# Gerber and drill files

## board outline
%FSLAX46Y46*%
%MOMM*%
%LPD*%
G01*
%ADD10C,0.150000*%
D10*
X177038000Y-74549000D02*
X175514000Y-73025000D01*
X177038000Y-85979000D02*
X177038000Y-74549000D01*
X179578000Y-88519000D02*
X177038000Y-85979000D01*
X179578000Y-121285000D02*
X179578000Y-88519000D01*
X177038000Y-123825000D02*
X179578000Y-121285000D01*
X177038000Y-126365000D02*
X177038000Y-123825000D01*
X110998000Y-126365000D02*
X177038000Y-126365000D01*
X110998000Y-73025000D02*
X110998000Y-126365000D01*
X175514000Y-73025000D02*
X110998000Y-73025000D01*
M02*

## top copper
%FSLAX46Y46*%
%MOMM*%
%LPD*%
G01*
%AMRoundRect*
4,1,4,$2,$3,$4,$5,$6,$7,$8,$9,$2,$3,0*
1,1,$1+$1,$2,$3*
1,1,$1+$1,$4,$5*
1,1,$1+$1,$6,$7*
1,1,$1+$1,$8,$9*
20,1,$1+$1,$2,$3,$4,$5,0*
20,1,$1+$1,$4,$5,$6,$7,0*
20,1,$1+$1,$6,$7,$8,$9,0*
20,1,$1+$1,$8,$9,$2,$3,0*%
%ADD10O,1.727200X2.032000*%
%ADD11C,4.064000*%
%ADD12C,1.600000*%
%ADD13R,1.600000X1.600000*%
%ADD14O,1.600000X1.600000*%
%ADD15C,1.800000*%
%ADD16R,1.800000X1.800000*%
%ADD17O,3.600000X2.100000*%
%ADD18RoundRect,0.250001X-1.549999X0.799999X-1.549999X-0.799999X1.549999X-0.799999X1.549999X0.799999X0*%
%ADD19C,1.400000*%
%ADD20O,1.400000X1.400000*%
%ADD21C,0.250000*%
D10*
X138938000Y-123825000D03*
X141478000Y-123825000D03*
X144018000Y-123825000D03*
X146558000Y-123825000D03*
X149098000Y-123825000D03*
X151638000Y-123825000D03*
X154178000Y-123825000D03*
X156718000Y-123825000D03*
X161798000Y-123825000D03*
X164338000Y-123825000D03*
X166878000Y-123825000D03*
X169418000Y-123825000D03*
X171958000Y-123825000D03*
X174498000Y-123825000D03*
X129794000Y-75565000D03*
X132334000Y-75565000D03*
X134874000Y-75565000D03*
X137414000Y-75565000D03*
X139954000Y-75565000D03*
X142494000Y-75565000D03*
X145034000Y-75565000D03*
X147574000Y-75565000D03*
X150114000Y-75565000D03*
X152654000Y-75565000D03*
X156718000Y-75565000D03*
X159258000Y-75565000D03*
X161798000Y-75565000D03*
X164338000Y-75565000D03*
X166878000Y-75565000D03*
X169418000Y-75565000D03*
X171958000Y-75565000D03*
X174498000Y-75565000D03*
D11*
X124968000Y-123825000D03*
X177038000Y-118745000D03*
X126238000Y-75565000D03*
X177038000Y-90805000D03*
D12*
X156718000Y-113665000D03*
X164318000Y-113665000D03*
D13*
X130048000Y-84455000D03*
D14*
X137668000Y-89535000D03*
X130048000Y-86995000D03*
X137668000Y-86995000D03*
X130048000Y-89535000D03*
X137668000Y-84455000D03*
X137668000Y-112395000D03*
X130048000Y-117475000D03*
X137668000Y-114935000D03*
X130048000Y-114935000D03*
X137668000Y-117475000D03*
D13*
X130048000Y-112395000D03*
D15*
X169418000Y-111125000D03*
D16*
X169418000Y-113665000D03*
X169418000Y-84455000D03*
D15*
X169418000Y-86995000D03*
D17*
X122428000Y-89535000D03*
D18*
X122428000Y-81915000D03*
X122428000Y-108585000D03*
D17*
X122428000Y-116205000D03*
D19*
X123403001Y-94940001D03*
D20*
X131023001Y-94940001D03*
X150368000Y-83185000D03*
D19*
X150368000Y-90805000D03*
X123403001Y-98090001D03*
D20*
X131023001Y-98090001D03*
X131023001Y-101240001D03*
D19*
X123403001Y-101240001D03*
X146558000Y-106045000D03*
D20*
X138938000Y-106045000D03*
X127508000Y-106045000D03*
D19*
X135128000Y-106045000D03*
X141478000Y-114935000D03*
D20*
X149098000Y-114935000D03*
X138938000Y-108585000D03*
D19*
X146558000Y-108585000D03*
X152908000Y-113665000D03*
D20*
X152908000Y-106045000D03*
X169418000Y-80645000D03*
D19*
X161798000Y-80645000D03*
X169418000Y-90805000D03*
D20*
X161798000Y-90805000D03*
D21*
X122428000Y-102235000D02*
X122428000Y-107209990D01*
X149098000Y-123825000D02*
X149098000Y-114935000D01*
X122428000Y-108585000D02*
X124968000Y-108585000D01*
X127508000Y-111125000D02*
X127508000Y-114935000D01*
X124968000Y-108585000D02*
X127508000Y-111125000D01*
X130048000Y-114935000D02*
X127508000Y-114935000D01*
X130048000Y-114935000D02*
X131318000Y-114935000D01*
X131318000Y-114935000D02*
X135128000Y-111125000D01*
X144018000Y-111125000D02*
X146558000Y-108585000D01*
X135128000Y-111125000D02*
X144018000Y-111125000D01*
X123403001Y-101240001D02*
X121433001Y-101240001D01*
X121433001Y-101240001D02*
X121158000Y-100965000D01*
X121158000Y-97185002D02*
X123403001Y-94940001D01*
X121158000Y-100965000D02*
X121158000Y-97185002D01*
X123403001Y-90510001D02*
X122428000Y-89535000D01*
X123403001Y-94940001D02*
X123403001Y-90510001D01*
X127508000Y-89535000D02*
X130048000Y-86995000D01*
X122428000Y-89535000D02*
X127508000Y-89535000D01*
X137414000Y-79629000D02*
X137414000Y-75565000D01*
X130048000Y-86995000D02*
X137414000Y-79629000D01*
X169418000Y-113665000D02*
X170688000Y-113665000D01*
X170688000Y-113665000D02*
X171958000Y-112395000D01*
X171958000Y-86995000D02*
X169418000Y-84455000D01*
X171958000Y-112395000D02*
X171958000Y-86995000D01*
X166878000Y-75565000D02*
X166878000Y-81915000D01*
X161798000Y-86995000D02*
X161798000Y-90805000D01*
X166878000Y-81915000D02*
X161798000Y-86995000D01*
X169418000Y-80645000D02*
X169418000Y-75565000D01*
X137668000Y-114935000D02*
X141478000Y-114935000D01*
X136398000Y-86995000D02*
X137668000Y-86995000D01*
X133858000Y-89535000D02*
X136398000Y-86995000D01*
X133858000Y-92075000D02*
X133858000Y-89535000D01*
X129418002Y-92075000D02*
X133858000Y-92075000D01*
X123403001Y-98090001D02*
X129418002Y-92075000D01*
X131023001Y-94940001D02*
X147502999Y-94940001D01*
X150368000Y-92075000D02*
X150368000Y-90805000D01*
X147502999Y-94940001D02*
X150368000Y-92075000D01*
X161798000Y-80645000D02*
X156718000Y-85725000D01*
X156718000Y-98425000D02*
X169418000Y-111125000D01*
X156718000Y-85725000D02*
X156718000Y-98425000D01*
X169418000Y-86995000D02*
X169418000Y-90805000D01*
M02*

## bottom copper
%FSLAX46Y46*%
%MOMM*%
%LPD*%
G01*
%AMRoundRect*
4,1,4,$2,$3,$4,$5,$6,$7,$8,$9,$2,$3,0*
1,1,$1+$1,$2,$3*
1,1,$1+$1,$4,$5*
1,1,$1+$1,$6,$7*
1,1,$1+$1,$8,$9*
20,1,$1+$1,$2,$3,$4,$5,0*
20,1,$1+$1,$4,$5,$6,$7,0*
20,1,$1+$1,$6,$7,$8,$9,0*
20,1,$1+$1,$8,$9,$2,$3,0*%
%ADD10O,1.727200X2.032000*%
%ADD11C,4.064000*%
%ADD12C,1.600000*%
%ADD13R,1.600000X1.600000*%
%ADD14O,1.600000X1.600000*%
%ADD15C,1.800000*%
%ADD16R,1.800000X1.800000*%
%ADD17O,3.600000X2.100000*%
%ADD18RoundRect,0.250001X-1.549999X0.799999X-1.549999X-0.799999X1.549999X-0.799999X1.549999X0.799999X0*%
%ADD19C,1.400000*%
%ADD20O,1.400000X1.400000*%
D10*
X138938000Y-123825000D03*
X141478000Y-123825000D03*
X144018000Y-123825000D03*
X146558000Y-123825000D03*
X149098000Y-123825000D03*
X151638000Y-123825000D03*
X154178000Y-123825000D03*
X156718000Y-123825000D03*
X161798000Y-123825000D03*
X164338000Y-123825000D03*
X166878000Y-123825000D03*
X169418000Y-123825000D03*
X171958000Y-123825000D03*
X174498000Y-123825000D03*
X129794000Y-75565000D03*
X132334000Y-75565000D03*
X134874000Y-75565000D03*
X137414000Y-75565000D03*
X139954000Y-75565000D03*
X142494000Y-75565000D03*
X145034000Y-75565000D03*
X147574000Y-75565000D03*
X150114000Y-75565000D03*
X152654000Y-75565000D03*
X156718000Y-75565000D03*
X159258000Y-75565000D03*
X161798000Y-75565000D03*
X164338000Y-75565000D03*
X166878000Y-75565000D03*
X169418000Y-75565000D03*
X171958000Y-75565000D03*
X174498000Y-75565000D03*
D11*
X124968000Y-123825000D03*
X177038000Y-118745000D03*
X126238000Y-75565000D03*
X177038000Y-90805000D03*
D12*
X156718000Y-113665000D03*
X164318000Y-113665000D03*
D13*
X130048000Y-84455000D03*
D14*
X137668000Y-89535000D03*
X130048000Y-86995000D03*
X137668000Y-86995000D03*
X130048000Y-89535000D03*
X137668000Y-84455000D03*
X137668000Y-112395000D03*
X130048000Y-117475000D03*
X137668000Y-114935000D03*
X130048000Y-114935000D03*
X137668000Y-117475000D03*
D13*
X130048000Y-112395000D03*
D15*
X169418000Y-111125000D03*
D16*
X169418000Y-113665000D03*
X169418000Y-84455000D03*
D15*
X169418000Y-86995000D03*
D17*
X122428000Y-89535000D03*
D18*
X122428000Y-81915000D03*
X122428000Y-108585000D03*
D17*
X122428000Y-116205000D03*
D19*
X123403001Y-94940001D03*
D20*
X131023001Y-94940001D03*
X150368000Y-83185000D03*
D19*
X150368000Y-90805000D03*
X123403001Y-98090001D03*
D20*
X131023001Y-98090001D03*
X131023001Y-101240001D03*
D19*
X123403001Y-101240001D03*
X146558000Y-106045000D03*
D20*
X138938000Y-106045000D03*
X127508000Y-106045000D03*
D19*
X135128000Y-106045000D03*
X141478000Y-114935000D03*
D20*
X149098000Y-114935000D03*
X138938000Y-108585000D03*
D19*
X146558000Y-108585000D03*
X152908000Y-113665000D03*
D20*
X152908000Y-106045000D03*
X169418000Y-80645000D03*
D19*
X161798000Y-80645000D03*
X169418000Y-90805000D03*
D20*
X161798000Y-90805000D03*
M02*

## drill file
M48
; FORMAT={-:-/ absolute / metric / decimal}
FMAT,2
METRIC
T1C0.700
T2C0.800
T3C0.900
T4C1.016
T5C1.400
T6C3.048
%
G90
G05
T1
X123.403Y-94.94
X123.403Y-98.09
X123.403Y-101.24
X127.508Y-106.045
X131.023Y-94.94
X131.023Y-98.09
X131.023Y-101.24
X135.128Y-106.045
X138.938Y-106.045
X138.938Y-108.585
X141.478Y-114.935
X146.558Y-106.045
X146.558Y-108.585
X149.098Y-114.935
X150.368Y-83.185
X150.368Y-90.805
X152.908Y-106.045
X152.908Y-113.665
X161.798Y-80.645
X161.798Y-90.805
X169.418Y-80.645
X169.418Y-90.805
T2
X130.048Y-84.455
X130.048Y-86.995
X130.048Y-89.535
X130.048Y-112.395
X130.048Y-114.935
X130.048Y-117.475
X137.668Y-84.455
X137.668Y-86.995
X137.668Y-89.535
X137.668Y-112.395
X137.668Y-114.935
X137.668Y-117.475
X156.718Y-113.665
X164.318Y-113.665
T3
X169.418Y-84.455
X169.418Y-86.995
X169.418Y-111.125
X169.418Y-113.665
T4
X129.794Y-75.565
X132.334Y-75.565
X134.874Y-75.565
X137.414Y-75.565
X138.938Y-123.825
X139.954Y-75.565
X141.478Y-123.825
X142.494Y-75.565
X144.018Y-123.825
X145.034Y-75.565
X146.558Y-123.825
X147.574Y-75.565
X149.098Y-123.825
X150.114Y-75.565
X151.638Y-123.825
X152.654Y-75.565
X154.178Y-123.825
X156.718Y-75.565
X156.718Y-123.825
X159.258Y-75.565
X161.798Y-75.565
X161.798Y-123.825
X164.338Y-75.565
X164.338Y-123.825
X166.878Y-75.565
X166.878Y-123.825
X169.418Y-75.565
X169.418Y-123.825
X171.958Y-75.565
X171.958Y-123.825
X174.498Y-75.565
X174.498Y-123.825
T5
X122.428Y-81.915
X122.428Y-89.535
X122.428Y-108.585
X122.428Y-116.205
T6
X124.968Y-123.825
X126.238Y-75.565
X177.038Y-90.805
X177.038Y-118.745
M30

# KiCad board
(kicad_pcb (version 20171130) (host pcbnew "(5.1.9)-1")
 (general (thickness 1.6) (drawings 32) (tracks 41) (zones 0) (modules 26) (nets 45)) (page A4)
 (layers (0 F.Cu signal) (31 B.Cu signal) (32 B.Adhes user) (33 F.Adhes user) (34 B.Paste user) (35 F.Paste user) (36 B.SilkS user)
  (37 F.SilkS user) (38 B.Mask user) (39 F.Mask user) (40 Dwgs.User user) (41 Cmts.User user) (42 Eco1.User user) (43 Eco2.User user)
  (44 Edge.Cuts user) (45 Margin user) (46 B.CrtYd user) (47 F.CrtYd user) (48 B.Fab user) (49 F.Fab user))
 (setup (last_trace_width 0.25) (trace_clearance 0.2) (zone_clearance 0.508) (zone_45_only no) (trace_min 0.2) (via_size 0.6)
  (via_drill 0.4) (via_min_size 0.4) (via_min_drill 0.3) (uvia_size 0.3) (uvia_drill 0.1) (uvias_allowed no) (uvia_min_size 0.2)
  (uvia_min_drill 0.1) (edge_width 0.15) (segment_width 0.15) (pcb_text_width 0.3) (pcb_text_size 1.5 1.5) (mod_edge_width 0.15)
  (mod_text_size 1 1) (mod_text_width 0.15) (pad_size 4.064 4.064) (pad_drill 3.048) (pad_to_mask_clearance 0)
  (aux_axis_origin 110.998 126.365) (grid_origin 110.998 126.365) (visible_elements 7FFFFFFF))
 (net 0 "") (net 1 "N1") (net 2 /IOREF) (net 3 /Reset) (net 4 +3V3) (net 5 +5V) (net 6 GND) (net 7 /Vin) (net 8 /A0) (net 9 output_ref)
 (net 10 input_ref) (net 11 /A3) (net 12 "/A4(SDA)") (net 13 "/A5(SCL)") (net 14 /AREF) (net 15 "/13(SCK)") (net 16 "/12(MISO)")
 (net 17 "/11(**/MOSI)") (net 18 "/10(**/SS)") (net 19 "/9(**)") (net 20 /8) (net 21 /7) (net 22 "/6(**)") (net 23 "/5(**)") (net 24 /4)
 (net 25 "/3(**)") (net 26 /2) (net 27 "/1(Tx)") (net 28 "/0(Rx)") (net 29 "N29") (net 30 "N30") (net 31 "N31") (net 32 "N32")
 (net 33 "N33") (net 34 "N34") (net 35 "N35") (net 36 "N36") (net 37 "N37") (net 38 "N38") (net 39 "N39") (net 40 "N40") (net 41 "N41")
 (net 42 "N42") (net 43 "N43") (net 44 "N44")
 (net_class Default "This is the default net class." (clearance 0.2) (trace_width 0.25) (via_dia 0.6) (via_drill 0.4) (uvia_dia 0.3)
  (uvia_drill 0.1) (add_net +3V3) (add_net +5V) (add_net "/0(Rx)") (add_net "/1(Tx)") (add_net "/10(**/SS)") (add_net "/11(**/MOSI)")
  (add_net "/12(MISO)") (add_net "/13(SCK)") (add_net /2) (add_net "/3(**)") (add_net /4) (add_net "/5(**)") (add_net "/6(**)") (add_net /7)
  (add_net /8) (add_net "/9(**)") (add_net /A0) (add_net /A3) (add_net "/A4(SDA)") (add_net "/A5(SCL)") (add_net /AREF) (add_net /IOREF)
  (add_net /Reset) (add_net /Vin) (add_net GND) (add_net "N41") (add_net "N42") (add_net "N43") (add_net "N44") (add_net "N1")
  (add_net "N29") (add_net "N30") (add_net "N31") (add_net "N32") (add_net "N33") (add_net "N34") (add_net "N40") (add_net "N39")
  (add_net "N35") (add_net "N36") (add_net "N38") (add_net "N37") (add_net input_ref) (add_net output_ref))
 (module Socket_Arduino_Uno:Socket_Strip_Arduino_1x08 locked (layer F.Cu) (at 138.938 123.825)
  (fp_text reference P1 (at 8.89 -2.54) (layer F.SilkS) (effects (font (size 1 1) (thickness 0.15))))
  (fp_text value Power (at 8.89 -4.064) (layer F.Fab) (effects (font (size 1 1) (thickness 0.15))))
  (pad 1 thru_hole oval (at 0 0) (size 1.7272 2.032) (drill 1.016) (layers *.Cu *.Mask F.SilkS) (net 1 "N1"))
  (pad 2 thru_hole oval (at 2.54 0) (size 1.7272 2.032) (drill 1.016) (layers *.Cu *.Mask F.SilkS) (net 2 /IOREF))
  (pad 3 thru_hole oval (at 5.08 0) (size 1.7272 2.032) (drill 1.016) (layers *.Cu *.Mask F.SilkS) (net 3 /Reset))
  (pad 4 thru_hole oval (at 7.62 0) (size 1.7272 2.032) (drill 1.016) (layers *.Cu *.Mask F.SilkS) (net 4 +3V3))
  (pad 5 thru_hole oval (at 10.16 0) (size 1.7272 2.032) (drill 1.016) (layers *.Cu *.Mask F.SilkS) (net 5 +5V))
  (pad 6 thru_hole oval (at 12.7 0) (size 1.7272 2.032) (drill 1.016) (layers *.Cu *.Mask F.SilkS) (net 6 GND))
  (pad 7 thru_hole oval (at 15.24 0) (size 1.7272 2.032) (drill 1.016) (layers *.Cu *.Mask F.SilkS) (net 6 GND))
  (pad 8 thru_hole oval (at 17.78 0) (size 1.7272 2.032) (drill 1.016) (layers *.Cu *.Mask F.SilkS) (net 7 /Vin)))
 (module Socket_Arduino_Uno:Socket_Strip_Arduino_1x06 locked (layer F.Cu) (at 161.798 123.825)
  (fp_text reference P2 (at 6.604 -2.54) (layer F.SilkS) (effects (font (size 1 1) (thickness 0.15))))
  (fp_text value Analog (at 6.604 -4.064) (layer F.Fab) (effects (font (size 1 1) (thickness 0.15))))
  (pad 1 thru_hole oval (at 0 0) (size 1.7272 2.032) (drill 1.016) (layers *.Cu *.Mask F.SilkS) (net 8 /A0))
  (pad 2 thru_hole oval (at 2.54 0) (size 1.7272 2.032) (drill 1.016) (layers *.Cu *.Mask F.SilkS) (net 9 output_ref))
  (pad 3 thru_hole oval (at 5.08 0) (size 1.7272 2.032) (drill 1.016) (layers *.Cu *.Mask F.SilkS) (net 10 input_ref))
  (pad 4 thru_hole oval (at 7.62 0) (size 1.7272 2.032) (drill 1.016) (layers *.Cu *.Mask F.SilkS) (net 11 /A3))
  (pad 5 thru_hole oval (at 10.16 0) (size 1.7272 2.032) (drill 1.016) (layers *.Cu *.Mask F.SilkS) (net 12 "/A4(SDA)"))
  (pad 6 thru_hole oval (at 12.7 0) (size 1.7272 2.032) (drill 1.016) (layers *.Cu *.Mask F.SilkS) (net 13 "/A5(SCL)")))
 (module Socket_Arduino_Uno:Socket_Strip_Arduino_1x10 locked (layer F.Cu) (at 129.794 75.565)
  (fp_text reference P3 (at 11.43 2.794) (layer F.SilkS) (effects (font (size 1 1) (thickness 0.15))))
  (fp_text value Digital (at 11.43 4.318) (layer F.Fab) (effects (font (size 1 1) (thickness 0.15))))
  (pad 1 thru_hole oval (at 0 0) (size 1.7272 2.032) (drill 1.016) (layers *.Cu *.Mask F.SilkS) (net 13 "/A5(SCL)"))
  (pad 2 thru_hole oval (at 2.54 0) (size 1.7272 2.032) (drill 1.016) (layers *.Cu *.Mask F.SilkS) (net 12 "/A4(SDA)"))
  (pad 3 thru_hole oval (at 5.08 0) (size 1.7272 2.032) (drill 1.016) (layers *.Cu *.Mask F.SilkS) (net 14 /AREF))
  (pad 4 thru_hole oval (at 7.62 0) (size 1.7272 2.032) (drill 1.016) (layers *.Cu *.Mask F.SilkS) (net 6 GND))
  (pad 5 thru_hole oval (at 10.16 0) (size 1.7272 2.032) (drill 1.016) (layers *.Cu *.Mask F.SilkS) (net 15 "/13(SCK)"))
  (pad 6 thru_hole oval (at 12.7 0) (size 1.7272 2.032) (drill 1.016) (layers *.Cu *.Mask F.SilkS) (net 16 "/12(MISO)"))
  (pad 7 thru_hole oval (at 15.24 0) (size 1.7272 2.032) (drill 1.016) (layers *.Cu *.Mask F.SilkS) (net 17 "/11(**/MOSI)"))
  (pad 8 thru_hole oval (at 17.78 0) (size 1.7272 2.032) (drill 1.016) (layers *.Cu *.Mask F.SilkS) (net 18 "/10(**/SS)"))
  (pad 9 thru_hole oval (at 20.32 0) (size 1.7272 2.032) (drill 1.016) (layers *.Cu *.Mask F.SilkS) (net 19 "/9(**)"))
  (pad 10 thru_hole oval (at 22.86 0) (size 1.7272 2.032) (drill 1.016) (layers *.Cu *.Mask F.SilkS) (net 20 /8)))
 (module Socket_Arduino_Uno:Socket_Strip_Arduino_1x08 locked (layer F.Cu) (at 156.718 75.565)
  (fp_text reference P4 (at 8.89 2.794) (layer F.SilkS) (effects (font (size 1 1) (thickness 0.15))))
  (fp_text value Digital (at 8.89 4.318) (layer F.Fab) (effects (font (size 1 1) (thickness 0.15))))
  (pad 1 thru_hole oval (at 0 0) (size 1.7272 2.032) (drill 1.016) (layers *.Cu *.Mask F.SilkS) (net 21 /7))
  (pad 2 thru_hole oval (at 2.54 0) (size 1.7272 2.032) (drill 1.016) (layers *.Cu *.Mask F.SilkS) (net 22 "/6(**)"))
  (pad 3 thru_hole oval (at 5.08 0) (size 1.7272 2.032) (drill 1.016) (layers *.Cu *.Mask F.SilkS) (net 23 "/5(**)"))
  (pad 4 thru_hole oval (at 7.62 0) (size 1.7272 2.032) (drill 1.016) (layers *.Cu *.Mask F.SilkS) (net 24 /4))
  (pad 5 thru_hole oval (at 10.16 0) (size 1.7272 2.032) (drill 1.016) (layers *.Cu *.Mask F.SilkS) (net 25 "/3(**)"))
  (pad 6 thru_hole oval (at 12.7 0) (size 1.7272 2.032) (drill 1.016) (layers *.Cu *.Mask F.SilkS) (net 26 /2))
  (pad 7 thru_hole oval (at 15.24 0) (size 1.7272 2.032) (drill 1.016) (layers *.Cu *.Mask F.SilkS) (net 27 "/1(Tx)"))
  (pad 8 thru_hole oval (at 17.78 0) (size 1.7272 2.032) (drill 1.016) (layers *.Cu *.Mask F.SilkS) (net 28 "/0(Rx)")))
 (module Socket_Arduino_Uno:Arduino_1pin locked (layer F.Cu) (at 124.968 123.825)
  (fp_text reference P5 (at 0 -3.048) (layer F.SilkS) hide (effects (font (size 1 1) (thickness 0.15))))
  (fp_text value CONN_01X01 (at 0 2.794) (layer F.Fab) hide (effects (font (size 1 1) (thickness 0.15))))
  (pad 1 thru_hole circle (at 0 0) (size 4.064 4.064) (drill 3.048) (layers *.Cu *.Mask F.SilkS) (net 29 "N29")))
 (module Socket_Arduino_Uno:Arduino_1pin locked (layer F.Cu) (at 177.038 118.745)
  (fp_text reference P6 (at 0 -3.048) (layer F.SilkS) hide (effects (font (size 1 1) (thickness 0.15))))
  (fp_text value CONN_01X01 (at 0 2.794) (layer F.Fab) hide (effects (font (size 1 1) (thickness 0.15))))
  (pad 1 thru_hole circle (at 0 0) (size 4.064 4.064) (drill 3.048) (layers *.Cu *.Mask F.SilkS) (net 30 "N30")))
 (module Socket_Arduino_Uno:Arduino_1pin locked (layer F.Cu) (at 126.238 75.565)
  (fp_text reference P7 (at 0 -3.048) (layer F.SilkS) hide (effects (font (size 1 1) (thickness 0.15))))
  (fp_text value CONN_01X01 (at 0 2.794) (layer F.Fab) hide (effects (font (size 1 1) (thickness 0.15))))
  (pad 1 thru_hole circle (at 0 0) (size 4.064 4.064) (drill 3.048) (layers *.Cu *.Mask F.SilkS) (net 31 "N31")))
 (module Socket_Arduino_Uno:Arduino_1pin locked (layer F.Cu) (at 177.038 90.805)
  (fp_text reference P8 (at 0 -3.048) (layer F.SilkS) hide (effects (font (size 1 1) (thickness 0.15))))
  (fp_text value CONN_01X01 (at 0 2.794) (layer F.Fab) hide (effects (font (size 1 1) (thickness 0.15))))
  (pad 1 thru_hole circle (at 0 0) (size 4.064 4.064) (drill 3.048) (layers *.Cu *.Mask F.SilkS) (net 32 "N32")))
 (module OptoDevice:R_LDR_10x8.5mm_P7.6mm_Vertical (layer F.Cu) (at 156.718 113.665)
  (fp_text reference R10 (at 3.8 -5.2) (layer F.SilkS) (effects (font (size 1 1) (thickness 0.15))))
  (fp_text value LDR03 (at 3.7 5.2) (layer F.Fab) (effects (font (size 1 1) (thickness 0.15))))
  (pad 1 thru_hole circle (at 0 0) (size 1.6 1.6) (drill 0.8) (layers *.Cu *.Mask) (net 11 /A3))
  (pad 2 thru_hole circle (at 7.6 0) (size 1.6 1.6) (drill 0.8) (layers *.Cu *.Mask) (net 6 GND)))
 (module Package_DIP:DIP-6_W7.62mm (layer F.Cu) (at 130.048 84.455)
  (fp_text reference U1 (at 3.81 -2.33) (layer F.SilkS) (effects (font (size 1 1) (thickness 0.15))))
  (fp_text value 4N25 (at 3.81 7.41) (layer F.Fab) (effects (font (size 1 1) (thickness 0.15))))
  (pad 1 thru_hole rect (at 0 0) (size 1.6 1.6) (drill 0.8) (layers *.Cu *.Mask) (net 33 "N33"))
  (pad 4 thru_hole oval (at 7.62 5.08) (size 1.6 1.6) (drill 0.8) (layers *.Cu *.Mask) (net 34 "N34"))
  (pad 2 thru_hole oval (at 0 2.54) (size 1.6 1.6) (drill 0.8) (layers *.Cu *.Mask) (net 6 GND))
  (pad 5 thru_hole oval (at 7.62 2.54) (size 1.6 1.6) (drill 0.8) (layers *.Cu *.Mask) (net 10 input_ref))
  (pad 3 thru_hole oval (at 0 5.08) (size 1.6 1.6) (drill 0.8) (layers *.Cu *.Mask) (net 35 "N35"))
  (pad 6 thru_hole oval (at 7.62 0) (size 1.6 1.6) (drill 0.8) (layers *.Cu *.Mask) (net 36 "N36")))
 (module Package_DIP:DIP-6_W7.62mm (layer F.Cu) (at 130.048 112.395)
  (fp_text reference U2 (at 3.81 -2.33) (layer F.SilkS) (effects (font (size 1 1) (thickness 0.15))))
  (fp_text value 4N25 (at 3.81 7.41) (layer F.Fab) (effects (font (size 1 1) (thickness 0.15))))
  (pad 6 thru_hole oval (at 7.62 0) (size 1.6 1.6) (drill 0.8) (layers *.Cu *.Mask) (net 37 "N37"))
  (pad 3 thru_hole oval (at 0 5.08) (size 1.6 1.6) (drill 0.8) (layers *.Cu *.Mask) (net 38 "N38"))
  (pad 5 thru_hole oval (at 7.62 2.54) (size 1.6 1.6) (drill 0.8) (layers *.Cu *.Mask) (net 9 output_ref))
  (pad 2 thru_hole oval (at 0 2.54) (size 1.6 1.6) (drill 0.8) (layers *.Cu *.Mask) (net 6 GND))
  (pad 4 thru_hole oval (at 7.62 5.08) (size 1.6 1.6) (drill 0.8) (layers *.Cu *.Mask) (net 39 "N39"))
  (pad 1 thru_hole rect (at 0 0) (size 1.6 1.6) (drill 0.8) (layers *.Cu *.Mask) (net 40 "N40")))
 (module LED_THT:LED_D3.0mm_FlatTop (layer F.Cu) (at 169.418 113.665 90)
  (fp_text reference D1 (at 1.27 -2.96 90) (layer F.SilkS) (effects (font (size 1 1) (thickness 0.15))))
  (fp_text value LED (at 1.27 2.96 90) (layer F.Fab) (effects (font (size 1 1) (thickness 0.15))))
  (pad 2 thru_hole circle (at 2.54 0 90) (size 1.8 1.8) (drill 0.9) (layers *.Cu *.Mask) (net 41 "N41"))
  (pad 1 thru_hole rect (at 0 0 90) (size 1.8 1.8) (drill 0.9) (layers *.Cu *.Mask) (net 6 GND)))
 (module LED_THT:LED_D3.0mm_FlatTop (layer F.Cu) (at 169.418 84.455 270)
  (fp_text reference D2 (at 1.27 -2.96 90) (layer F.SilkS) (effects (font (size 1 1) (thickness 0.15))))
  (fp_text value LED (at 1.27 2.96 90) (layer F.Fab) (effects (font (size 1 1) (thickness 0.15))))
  (pad 1 thru_hole rect (at 0 0 270) (size 1.8 1.8) (drill 0.9) (layers *.Cu *.Mask) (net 6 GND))
  (pad 2 thru_hole circle (at 2.54 0 270) (size 1.8 1.8) (drill 0.9) (layers *.Cu *.Mask) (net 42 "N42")))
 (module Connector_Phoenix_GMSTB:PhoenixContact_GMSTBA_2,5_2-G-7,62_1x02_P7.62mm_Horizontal (layer F.Cu) (at 122.428 81.915 270)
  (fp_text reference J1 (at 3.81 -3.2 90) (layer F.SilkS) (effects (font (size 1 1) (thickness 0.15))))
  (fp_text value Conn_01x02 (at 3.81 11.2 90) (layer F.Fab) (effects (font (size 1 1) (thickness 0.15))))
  (pad 2 thru_hole oval (at 7.62 0 270) (size 2.1 3.6) (drill 1.4) (layers *.Cu *.Mask) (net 6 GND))
  (pad 1 thru_hole roundrect (at 0 0 270) (size 2.1 3.6) (drill 1.4) (layers *.Cu *.Mask) (roundrect_rratio 0.119048) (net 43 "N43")))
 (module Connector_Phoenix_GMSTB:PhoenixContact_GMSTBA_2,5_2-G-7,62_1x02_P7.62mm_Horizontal (layer F.Cu) (at 122.428 108.585 270)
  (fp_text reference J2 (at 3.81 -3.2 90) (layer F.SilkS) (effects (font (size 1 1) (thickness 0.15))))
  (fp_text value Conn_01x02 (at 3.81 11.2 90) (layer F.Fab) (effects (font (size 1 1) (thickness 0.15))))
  (pad 1 thru_hole roundrect (at 0 0 270) (size 2.1 3.6) (drill 1.4) (layers *.Cu *.Mask) (roundrect_rratio 0.119048) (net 6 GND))
  (pad 2 thru_hole oval (at 7.62 0 270) (size 2.1 3.6) (drill 1.4) (layers *.Cu *.Mask) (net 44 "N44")))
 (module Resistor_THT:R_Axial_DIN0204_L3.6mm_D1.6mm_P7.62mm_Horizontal (layer F.Cu) (at 123.403001 94.940001)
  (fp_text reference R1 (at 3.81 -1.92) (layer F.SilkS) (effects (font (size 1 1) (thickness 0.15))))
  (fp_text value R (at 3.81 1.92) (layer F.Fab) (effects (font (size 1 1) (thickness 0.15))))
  (pad 1 thru_hole circle (at 0 0) (size 1.4 1.4) (drill 0.7) (layers *.Cu *.Mask) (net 6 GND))
  (pad 2 thru_hole oval (at 7.62 0) (size 1.4 1.4) (drill 0.7) (layers *.Cu *.Mask) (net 33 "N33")))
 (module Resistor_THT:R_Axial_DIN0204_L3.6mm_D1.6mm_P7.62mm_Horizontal (layer F.Cu) (at 150.368 90.805 90)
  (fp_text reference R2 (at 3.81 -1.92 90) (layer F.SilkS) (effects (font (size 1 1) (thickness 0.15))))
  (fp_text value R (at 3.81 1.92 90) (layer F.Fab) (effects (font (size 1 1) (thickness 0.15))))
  (pad 2 thru_hole oval (at 7.62 0 90) (size 1.4 1.4) (drill 0.7) (layers *.Cu *.Mask) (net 43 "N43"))
  (pad 1 thru_hole circle (at 0 0 90) (size 1.4 1.4) (drill 0.7) (layers *.Cu *.Mask) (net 33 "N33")))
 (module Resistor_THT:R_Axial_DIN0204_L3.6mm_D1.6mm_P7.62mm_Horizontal (layer F.Cu) (at 123.403001 98.090001)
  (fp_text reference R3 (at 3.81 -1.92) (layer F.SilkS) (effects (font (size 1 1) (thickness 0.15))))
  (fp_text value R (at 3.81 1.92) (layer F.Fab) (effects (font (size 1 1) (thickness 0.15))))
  (pad 1 thru_hole circle (at 0 0) (size 1.4 1.4) (drill 0.7) (layers *.Cu *.Mask) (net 10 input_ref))
  (pad 2 thru_hole oval (at 7.62 0) (size 1.4 1.4) (drill 0.7) (layers *.Cu *.Mask) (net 5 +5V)))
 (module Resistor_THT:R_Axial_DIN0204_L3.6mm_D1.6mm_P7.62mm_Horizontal (layer F.Cu) (at 123.403001 101.240001)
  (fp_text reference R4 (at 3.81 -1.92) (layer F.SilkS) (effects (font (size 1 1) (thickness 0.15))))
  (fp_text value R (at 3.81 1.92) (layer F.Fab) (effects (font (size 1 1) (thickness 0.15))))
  (pad 2 thru_hole oval (at 7.62 0) (size 1.4 1.4) (drill 0.7) (layers *.Cu *.Mask) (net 34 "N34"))
  (pad 1 thru_hole circle (at 0 0) (size 1.4 1.4) (drill 0.7) (layers *.Cu *.Mask) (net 6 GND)))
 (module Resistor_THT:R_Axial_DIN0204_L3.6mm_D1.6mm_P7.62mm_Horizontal (layer F.Cu) (at 146.558 106.045 180)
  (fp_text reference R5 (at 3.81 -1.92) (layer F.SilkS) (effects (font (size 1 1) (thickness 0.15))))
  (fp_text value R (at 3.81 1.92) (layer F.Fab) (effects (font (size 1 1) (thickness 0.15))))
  (pad 1 thru_hole circle (at 0 0 180) (size 1.4 1.4) (drill 0.7) (layers *.Cu *.Mask) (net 6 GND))
  (pad 2 thru_hole oval (at 7.62 0 180) (size 1.4 1.4) (drill 0.7) (layers *.Cu *.Mask) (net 40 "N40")))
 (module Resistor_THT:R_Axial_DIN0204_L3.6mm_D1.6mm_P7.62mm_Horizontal (layer F.Cu) (at 135.128 106.045 180)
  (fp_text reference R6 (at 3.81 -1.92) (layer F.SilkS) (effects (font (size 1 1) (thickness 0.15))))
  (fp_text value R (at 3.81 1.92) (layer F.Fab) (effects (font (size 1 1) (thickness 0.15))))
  (pad 2 thru_hole oval (at 7.62 0 180) (size 1.4 1.4) (drill 0.7) (layers *.Cu *.Mask) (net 44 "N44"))
  (pad 1 thru_hole circle (at 0 0 180) (size 1.4 1.4) (drill 0.7) (layers *.Cu *.Mask) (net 40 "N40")))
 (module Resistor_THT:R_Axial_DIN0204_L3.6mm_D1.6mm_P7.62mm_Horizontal (layer F.Cu) (at 141.478 114.935)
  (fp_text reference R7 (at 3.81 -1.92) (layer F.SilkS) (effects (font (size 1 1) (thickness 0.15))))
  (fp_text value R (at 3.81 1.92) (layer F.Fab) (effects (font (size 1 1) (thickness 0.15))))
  (pad 1 thru_hole circle (at 0 0) (size 1.4 1.4) (drill 0.7) (layers *.Cu *.Mask) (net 9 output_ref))
  (pad 2 thru_hole oval (at 7.62 0) (size 1.4 1.4) (drill 0.7) (layers *.Cu *.Mask) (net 5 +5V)))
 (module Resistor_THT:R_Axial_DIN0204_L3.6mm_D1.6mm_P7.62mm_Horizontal (layer F.Cu) (at 146.558 108.585 180)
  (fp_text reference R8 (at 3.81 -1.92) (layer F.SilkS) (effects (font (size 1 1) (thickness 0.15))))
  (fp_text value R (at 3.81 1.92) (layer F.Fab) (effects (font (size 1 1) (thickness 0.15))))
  (pad 2 thru_hole oval (at 7.62 0 180) (size 1.4 1.4) (drill 0.7) (layers *.Cu *.Mask) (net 39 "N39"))
  (pad 1 thru_hole circle (at 0 0 180) (size 1.4 1.4) (drill 0.7) (layers *.Cu *.Mask) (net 6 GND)))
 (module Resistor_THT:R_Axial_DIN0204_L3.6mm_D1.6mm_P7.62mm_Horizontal (layer F.Cu) (at 152.908 113.665 90)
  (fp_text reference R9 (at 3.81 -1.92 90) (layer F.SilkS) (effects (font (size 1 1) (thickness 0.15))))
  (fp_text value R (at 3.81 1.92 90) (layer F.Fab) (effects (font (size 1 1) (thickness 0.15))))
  (pad 1 thru_hole circle (at 0 0 90) (size 1.4 1.4) (drill 0.7) (layers *.Cu *.Mask) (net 11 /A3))
  (pad 2 thru_hole oval (at 7.62 0 90) (size 1.4 1.4) (drill 0.7) (layers *.Cu *.Mask) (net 5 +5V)))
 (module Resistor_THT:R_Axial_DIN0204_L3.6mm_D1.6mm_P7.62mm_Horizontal (layer F.Cu) (at 161.798 80.645)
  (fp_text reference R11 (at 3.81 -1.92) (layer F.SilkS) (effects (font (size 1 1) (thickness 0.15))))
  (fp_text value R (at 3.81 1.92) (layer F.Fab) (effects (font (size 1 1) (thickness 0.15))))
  (pad 2 thru_hole oval (at 7.62 0) (size 1.4 1.4) (drill 0.7) (layers *.Cu *.Mask) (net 26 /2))
  (pad 1 thru_hole circle (at 0 0) (size 1.4 1.4) (drill 0.7) (layers *.Cu *.Mask) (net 41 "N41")))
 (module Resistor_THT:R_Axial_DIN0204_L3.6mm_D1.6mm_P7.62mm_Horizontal (layer F.Cu) (at 169.418 90.805 180)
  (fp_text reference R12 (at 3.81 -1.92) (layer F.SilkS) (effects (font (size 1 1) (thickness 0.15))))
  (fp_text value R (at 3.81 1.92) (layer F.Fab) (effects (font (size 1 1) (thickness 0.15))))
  (pad 1 thru_hole circle (at 0 0 180) (size 1.4 1.4) (drill 0.7) (layers *.Cu *.Mask) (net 42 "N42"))
  (pad 2 thru_hole oval (at 7.62 0 180) (size 1.4 1.4) (drill 0.7) (layers *.Cu *.Mask) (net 25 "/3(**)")))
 (gr_line (start 177.038 74.549) (end 175.514 73.025) (angle 90) (layer Edge.Cuts) (width 0.15))
 (gr_line (start 177.038 85.979) (end 177.038 74.549) (angle 90) (layer Edge.Cuts) (width 0.15))
 (gr_line (start 179.578 88.519) (end 177.038 85.979) (angle 90) (layer Edge.Cuts) (width 0.15))
 (gr_line (start 179.578 121.285) (end 179.578 88.519) (angle 90) (layer Edge.Cuts) (width 0.15))
 (gr_line (start 177.038 123.825) (end 179.578 121.285) (angle 90) (layer Edge.Cuts) (width 0.15))
 (gr_line (start 177.038 126.365) (end 177.038 123.825) (angle 90) (layer Edge.Cuts) (width 0.15))
 (gr_line (start 110.998 126.365) (end 177.038 126.365) (angle 90) (layer Edge.Cuts) (width 0.15))
 (gr_line (start 110.998 73.025) (end 110.998 126.365) (angle 90) (layer Edge.Cuts) (width 0.15))
 (gr_line (start 175.514 73.025) (end 110.998 73.025) (angle 90) (layer Edge.Cuts) (width 0.15))
 (segment (start 122.428 102.235) (end 122.428 107.20999) (width 0.25) (layer F.Cu) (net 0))
 (segment (start 149.098 123.825) (end 149.098 114.935) (width 0.25) (layer F.Cu) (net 5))
 (segment (start 122.428 108.585) (end 124.968 108.585) (width 0.25) (layer F.Cu) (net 6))
 (segment (start 127.508 111.125) (end 127.508 114.935) (width 0.25) (layer F.Cu) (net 6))
 (segment (start 124.968 108.585) (end 127.508 111.125) (width 0.25) (layer F.Cu) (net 6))
 (segment (start 130.048 114.935) (end 127.508 114.935) (width 0.25) (layer F.Cu) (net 6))
 (segment (start 130.048 114.935) (end 131.318 114.935) (width 0.25) (layer F.Cu) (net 6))
 (segment (start 131.318 114.935) (end 135.128 111.125) (width 0.25) (layer F.Cu) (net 6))
 (segment (start 144.018 111.125) (end 146.558 108.585) (width 0.25) (layer F.Cu) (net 6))
 (segment (start 135.128 111.125) (end 144.018 111.125) (width 0.25) (layer F.Cu) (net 6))
 (segment (start 123.403001 101.240001) (end 121.433001 101.240001) (width 0.25) (layer F.Cu) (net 6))
 (segment (start 121.433001 101.240001) (end 121.158 100.965) (width 0.25) (layer F.Cu) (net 6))
 (segment (start 121.158 97.185002) (end 123.403001 94.940001) (width 0.25) (layer F.Cu) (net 6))
 (segment (start 121.158 100.965) (end 121.158 97.185002) (width 0.25) (layer F.Cu) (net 6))
 (segment (start 123.403001 90.510001) (end 122.428 89.535) (width 0.25) (layer F.Cu) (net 6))
 (segment (start 123.403001 94.940001) (end 123.403001 90.510001) (width 0.25) (layer F.Cu) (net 6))
 (segment (start 127.508 89.535) (end 130.048 86.995) (width 0.25) (layer F.Cu) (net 6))
 (segment (start 122.428 89.535) (end 127.508 89.535) (width 0.25) (layer F.Cu) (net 6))
 (segment (start 137.414 79.629) (end 137.414 75.565) (width 0.25) (layer F.Cu) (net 6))
 (segment (start 130.048 86.995) (end 137.414 79.629) (width 0.25) (layer F.Cu) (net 6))
 (segment (start 169.418 113.665) (end 170.688 113.665) (width 0.25) (layer F.Cu) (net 6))
 (segment (start 170.688 113.665) (end 171.958 112.395) (width 0.25) (layer F.Cu) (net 6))
 (segment (start 171.958 86.995) (end 169.418 84.455) (width 0.25) (layer F.Cu) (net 6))
 (segment (start 171.958 112.395) (end 171.958 86.995) (width 0.25) (layer F.Cu) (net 6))
 (segment (start 166.878 75.565) (end 166.878 81.915) (width 0.25) (layer F.Cu) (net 25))
 (segment (start 161.798 86.995) (end 161.798 90.805) (width 0.25) (layer F.Cu) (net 25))
 (segment (start 166.878 81.915) (end 161.798 86.995) (width 0.25) (layer F.Cu) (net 25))
 (segment (start 169.418 80.645) (end 169.418 75.565) (width 0.25) (layer F.Cu) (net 26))
 (segment (start 137.668 114.935) (end 141.478 114.935) (width 0.25) (layer F.Cu) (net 9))
 (segment (start 136.398 86.995) (end 137.668 86.995) (width 0.25) (layer F.Cu) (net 10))
 (segment (start 133.858 89.535) (end 136.398 86.995) (width 0.25) (layer F.Cu) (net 10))
 (segment (start 133.858 92.075) (end 133.858 89.535) (width 0.25) (layer F.Cu) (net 10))
 (segment (start 129.418002 92.075) (end 133.858 92.075) (width 0.25) (layer F.Cu) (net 10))
 (segment (start 123.403001 98.090001) (end 129.418002 92.075) (width 0.25) (layer F.Cu) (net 10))
 (segment (start 131.023001 94.940001) (end 147.502999 94.940001) (width 0.25) (layer F.Cu) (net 33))
 (segment (start 150.368 92.075) (end 150.368 90.805) (width 0.25) (layer F.Cu) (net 33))
 (segment (start 147.502999 94.940001) (end 150.368 92.075) (width 0.25) (layer F.Cu) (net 33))
 (segment (start 161.798 80.645) (end 156.718 85.725) (width 0.25) (layer F.Cu) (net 41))
 (segment (start 156.718 98.425) (end 169.418 111.125) (width 0.25) (layer F.Cu) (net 41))
 (segment (start 156.718 85.725) (end 156.718 98.425) (width 0.25) (layer F.Cu) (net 41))
 (segment (start 169.418 86.995) (end 169.418 90.805) (width 0.25) (layer F.Cu) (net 42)))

